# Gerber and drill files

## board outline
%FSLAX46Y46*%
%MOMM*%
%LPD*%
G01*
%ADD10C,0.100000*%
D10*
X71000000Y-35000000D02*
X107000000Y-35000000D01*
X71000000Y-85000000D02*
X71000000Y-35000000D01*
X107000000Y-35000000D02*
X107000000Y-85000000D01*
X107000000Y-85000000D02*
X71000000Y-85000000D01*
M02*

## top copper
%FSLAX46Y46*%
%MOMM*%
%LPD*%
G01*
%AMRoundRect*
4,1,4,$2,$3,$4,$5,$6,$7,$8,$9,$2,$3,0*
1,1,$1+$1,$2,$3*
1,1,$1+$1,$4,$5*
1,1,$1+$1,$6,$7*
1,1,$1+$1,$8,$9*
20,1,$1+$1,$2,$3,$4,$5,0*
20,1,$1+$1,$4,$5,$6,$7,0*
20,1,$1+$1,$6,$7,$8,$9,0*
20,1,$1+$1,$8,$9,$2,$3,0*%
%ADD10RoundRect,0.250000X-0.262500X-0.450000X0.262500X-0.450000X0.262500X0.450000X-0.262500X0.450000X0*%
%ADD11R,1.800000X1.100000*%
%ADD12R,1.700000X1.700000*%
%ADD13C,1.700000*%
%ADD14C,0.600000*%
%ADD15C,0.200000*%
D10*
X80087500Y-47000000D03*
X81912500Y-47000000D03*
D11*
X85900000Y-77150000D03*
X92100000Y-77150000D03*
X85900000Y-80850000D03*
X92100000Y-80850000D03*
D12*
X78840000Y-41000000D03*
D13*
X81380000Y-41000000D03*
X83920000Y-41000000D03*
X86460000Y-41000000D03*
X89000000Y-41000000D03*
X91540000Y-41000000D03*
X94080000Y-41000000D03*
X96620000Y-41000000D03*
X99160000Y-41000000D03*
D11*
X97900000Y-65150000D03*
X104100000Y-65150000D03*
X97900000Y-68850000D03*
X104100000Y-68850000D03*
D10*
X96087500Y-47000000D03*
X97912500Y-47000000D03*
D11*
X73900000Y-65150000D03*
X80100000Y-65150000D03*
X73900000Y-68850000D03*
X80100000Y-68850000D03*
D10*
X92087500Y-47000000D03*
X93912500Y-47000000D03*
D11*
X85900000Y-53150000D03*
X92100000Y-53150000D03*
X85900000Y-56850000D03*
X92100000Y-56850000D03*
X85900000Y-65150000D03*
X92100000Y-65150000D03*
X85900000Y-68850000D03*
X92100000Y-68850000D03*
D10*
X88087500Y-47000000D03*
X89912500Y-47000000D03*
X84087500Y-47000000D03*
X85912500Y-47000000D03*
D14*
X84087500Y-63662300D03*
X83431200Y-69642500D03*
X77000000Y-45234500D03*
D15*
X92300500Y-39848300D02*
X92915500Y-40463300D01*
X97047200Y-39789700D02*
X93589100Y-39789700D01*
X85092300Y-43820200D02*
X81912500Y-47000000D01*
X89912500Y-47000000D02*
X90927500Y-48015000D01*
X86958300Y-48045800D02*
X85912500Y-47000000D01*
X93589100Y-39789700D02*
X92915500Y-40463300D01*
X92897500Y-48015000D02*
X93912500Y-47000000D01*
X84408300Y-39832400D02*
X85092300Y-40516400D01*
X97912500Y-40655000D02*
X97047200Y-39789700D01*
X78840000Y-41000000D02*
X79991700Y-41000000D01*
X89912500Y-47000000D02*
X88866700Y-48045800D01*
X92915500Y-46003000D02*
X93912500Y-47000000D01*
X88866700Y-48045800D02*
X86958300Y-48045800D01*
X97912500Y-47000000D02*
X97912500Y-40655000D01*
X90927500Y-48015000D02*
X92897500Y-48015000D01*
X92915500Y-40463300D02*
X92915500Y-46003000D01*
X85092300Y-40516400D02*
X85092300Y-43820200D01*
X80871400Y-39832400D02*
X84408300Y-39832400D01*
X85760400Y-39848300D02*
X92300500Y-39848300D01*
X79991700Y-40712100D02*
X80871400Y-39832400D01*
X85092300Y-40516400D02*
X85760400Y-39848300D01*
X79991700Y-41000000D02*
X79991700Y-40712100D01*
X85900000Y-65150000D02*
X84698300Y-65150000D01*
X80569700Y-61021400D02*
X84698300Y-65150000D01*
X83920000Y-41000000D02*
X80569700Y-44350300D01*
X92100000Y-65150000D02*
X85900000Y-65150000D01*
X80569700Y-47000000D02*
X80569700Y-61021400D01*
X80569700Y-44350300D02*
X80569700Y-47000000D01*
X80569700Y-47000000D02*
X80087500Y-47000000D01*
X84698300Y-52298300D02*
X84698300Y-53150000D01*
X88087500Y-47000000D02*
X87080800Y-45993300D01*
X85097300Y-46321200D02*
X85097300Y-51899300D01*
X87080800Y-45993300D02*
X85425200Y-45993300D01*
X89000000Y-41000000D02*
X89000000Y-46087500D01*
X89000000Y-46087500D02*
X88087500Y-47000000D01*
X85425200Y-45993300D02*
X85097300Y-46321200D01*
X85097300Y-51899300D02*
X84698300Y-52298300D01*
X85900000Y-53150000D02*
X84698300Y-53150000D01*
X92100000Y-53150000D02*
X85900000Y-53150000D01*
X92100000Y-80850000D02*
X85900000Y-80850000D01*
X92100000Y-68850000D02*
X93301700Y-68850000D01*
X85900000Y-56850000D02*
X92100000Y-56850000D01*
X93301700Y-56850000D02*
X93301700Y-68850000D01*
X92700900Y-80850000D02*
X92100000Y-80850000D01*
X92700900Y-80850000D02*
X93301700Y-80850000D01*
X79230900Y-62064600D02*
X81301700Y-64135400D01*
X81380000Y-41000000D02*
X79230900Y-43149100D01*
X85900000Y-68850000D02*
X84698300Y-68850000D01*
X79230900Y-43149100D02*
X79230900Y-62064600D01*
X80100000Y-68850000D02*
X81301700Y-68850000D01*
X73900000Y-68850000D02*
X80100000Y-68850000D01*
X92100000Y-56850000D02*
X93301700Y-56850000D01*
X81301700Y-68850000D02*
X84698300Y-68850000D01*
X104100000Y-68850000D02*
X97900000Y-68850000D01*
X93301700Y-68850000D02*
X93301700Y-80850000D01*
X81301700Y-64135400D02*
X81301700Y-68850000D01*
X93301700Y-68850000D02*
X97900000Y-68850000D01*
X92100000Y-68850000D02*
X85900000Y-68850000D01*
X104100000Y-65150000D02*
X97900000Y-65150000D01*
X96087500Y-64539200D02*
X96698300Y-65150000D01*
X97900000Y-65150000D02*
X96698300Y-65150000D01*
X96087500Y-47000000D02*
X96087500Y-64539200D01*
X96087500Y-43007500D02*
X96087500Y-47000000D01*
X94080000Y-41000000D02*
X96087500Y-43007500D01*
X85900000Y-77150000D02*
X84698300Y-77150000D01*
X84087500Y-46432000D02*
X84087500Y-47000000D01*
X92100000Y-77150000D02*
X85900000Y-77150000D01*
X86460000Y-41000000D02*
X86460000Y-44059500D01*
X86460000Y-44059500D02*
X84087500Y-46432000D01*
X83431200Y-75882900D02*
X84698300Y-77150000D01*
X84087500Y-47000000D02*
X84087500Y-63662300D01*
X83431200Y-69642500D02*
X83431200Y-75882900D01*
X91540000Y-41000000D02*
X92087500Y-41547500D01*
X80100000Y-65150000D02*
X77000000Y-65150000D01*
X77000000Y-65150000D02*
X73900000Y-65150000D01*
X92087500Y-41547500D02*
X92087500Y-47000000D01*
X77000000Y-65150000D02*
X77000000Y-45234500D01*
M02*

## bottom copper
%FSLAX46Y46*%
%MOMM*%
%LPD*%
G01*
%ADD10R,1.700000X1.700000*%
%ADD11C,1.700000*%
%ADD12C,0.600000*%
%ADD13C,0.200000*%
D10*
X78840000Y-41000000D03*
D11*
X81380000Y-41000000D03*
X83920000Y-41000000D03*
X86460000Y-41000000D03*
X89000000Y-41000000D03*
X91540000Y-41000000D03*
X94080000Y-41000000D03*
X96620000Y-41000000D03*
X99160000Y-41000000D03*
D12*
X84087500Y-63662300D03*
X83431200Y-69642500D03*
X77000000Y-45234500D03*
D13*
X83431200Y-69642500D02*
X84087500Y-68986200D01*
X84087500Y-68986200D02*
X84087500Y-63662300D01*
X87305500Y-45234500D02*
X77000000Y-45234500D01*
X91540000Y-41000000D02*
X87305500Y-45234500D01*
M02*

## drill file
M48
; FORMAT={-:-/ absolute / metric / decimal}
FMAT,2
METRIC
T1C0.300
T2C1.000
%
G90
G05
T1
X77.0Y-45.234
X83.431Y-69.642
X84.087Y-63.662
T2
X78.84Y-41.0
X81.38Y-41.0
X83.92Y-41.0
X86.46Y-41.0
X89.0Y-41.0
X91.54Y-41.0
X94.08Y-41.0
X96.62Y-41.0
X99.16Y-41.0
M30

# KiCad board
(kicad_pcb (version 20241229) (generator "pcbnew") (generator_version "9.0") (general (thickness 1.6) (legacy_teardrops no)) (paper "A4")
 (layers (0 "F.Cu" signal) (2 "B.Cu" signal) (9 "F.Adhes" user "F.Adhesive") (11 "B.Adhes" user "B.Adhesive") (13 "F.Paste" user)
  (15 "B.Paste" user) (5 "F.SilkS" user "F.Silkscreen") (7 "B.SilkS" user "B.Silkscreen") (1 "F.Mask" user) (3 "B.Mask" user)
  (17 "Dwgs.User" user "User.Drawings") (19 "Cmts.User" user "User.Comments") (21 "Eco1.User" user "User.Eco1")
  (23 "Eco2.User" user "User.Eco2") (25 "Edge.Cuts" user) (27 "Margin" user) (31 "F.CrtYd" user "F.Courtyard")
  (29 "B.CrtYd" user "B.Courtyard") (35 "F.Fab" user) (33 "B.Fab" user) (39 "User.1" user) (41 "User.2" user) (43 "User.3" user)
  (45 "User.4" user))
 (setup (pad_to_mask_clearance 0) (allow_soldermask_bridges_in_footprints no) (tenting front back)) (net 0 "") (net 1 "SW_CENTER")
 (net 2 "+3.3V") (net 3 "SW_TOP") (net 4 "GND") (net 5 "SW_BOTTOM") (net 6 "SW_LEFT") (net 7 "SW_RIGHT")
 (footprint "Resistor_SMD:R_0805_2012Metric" (layer "F.Cu") (at 81 47)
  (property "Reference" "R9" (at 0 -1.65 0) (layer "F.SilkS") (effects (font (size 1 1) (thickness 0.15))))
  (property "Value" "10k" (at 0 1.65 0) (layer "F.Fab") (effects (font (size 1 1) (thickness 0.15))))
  (pad "1" smd roundrect (at -0.9125 0) (size 1.025 1.4) (layers "F.Cu" "F.Mask" "F.Paste") (roundrect_rratio 0.243902) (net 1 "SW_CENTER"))
  (pad "2" smd roundrect (at 0.9125 0) (size 1.025 1.4) (layers "F.Cu" "F.Mask" "F.Paste") (roundrect_rratio 0.243902) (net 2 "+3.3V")))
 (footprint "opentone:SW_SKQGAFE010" (layer "F.Cu") (at 89 79)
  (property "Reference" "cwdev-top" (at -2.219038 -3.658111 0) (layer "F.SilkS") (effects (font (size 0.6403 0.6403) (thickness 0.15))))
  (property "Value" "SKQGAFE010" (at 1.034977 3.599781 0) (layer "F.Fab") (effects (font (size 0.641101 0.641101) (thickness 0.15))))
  (pad "1" smd rect (at -3.1 -1.85) (size 1.8 1.1) (layers "F.Cu" "F.Mask" "F.Paste") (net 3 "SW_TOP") (solder_mask_margin 0.102))
  (pad "2" smd rect (at 3.1 -1.85) (size 1.8 1.1) (layers "F.Cu" "F.Mask" "F.Paste") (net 3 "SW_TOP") (solder_mask_margin 0.102))
  (pad "3" smd rect (at -3.1 1.85) (size 1.8 1.1) (layers "F.Cu" "F.Mask" "F.Paste") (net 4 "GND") (solder_mask_margin 0.102))
  (pad "4" smd rect (at 3.1 1.85) (size 1.8 1.1) (layers "F.Cu" "F.Mask" "F.Paste") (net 4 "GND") (solder_mask_margin 0.102))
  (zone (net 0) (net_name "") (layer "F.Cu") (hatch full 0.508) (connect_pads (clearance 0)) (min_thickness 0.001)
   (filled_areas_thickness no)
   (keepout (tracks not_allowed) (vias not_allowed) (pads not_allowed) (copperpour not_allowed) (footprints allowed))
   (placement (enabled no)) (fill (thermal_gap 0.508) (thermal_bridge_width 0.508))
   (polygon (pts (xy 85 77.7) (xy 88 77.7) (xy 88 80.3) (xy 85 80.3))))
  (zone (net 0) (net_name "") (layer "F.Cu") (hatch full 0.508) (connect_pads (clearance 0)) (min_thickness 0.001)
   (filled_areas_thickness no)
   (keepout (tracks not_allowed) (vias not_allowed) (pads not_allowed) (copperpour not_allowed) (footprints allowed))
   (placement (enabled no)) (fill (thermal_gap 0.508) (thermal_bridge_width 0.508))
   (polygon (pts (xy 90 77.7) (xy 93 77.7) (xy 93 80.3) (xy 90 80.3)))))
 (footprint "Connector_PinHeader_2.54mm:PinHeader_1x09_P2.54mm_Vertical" (layer "F.Cu") (at 78.84 41 90)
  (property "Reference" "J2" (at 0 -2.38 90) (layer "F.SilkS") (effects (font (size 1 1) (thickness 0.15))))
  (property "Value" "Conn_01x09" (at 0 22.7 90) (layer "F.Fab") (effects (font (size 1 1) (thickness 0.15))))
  (pad "1" thru_hole rect (at 0 0 90) (size 1.7 1.7) (drill 1) (layers "*.Cu" "*.Mask") (remove_unused_layers no) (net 2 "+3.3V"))
  (pad "2" thru_hole circle (at 0 2.54 90) (size 1.7 1.7) (drill 1) (layers "*.Cu" "*.Mask") (remove_unused_layers no) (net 4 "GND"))
  (pad "3" thru_hole circle (at 0 5.08 90) (size 1.7 1.7) (drill 1) (layers "*.Cu" "*.Mask") (remove_unused_layers no) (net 1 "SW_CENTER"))
  (pad "4" thru_hole circle (at 0 7.62 90) (size 1.7 1.7) (drill 1) (layers "*.Cu" "*.Mask") (remove_unused_layers no) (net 3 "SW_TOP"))
  (pad "5" thru_hole circle (at 0 10.16 90) (size 1.7 1.7) (drill 1) (layers "*.Cu" "*.Mask") (remove_unused_layers no) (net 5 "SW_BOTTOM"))
  (pad "6" thru_hole circle (at 0 12.7 90) (size 1.7 1.7) (drill 1) (layers "*.Cu" "*.Mask") (remove_unused_layers no) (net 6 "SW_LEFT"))
  (pad "7" thru_hole circle (at 0 15.24 90) (size 1.7 1.7) (drill 1) (layers "*.Cu" "*.Mask") (remove_unused_layers no) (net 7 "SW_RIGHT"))
  (pad "8" thru_hole circle (at 0 17.78 90) (size 1.7 1.7) (drill 1) (layers "*.Cu" "*.Mask") (remove_unused_layers no))
  (pad "9" thru_hole circle (at 0 20.32 90) (size 1.7 1.7) (drill 1) (layers "*.Cu" "*.Mask") (remove_unused_layers no)))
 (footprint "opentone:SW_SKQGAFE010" (layer "F.Cu") (at 101 67)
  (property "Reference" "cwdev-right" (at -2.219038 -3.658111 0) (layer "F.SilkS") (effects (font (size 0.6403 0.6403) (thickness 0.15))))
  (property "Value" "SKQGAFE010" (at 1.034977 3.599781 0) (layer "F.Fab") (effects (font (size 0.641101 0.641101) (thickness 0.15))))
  (pad "1" smd rect (at -3.1 -1.85) (size 1.8 1.1) (layers "F.Cu" "F.Mask" "F.Paste") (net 7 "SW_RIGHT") (solder_mask_margin 0.102))
  (pad "2" smd rect (at 3.1 -1.85) (size 1.8 1.1) (layers "F.Cu" "F.Mask" "F.Paste") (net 7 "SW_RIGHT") (solder_mask_margin 0.102))
  (pad "3" smd rect (at -3.1 1.85) (size 1.8 1.1) (layers "F.Cu" "F.Mask" "F.Paste") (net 4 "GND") (solder_mask_margin 0.102))
  (pad "4" smd rect (at 3.1 1.85) (size 1.8 1.1) (layers "F.Cu" "F.Mask" "F.Paste") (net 4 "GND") (solder_mask_margin 0.102))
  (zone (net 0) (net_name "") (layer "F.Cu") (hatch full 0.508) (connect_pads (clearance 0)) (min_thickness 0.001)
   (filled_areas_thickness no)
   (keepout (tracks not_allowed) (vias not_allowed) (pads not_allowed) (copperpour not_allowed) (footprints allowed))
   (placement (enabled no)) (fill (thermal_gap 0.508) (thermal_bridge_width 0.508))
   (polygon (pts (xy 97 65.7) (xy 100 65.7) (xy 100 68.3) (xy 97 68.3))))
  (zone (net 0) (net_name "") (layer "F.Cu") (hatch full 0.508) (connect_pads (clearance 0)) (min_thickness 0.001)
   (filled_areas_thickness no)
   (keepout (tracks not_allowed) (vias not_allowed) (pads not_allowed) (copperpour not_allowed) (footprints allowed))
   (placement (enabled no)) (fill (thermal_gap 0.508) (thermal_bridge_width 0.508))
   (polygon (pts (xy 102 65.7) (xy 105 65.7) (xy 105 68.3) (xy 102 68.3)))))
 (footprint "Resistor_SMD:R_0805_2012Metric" (layer "F.Cu") (at 97 47)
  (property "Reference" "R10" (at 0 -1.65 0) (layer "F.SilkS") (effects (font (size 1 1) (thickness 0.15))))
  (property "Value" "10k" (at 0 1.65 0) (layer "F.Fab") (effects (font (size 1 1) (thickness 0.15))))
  (pad "1" smd roundrect (at -0.9125 0) (size 1.025 1.4) (layers "F.Cu" "F.Mask" "F.Paste") (roundrect_rratio 0.243902) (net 7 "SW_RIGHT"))
  (pad "2" smd roundrect (at 0.9125 0) (size 1.025 1.4) (layers "F.Cu" "F.Mask" "F.Paste") (roundrect_rratio 0.243902) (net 2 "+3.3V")))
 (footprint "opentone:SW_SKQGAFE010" (layer "F.Cu") (at 77 67)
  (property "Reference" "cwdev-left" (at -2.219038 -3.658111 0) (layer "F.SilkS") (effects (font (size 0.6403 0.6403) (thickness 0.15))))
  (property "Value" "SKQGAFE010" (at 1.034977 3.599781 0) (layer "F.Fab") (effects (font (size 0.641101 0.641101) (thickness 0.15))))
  (pad "1" smd rect (at -3.1 -1.85) (size 1.8 1.1) (layers "F.Cu" "F.Mask" "F.Paste") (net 6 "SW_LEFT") (solder_mask_margin 0.102))
  (pad "2" smd rect (at 3.1 -1.85) (size 1.8 1.1) (layers "F.Cu" "F.Mask" "F.Paste") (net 6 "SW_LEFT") (solder_mask_margin 0.102))
  (pad "3" smd rect (at -3.1 1.85) (size 1.8 1.1) (layers "F.Cu" "F.Mask" "F.Paste") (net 4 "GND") (solder_mask_margin 0.102))
  (pad "4" smd rect (at 3.1 1.85) (size 1.8 1.1) (layers "F.Cu" "F.Mask" "F.Paste") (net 4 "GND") (solder_mask_margin 0.102))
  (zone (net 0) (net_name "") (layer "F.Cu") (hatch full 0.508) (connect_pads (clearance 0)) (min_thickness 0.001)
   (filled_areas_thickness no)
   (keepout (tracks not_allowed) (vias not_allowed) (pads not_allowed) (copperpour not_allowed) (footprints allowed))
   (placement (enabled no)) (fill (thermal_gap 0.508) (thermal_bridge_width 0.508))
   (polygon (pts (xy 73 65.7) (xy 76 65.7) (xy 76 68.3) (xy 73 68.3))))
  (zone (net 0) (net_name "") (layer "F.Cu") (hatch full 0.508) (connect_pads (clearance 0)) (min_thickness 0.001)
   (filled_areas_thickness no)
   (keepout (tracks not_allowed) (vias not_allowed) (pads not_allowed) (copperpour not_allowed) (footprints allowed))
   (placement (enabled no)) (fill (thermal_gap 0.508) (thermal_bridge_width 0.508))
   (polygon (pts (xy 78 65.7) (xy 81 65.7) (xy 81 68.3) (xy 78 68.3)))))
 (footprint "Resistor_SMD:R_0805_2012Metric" (layer "F.Cu") (at 93 47)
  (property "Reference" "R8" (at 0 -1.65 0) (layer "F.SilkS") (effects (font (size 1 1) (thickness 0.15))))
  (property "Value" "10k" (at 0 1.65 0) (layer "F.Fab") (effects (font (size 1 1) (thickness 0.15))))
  (pad "1" smd roundrect (at -0.9125 0) (size 1.025 1.4) (layers "F.Cu" "F.Mask" "F.Paste") (roundrect_rratio 0.243902) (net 6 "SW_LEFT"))
  (pad "2" smd roundrect (at 0.9125 0) (size 1.025 1.4) (layers "F.Cu" "F.Mask" "F.Paste") (roundrect_rratio 0.243902) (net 2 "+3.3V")))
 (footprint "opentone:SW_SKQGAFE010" (layer "F.Cu") (at 89 55)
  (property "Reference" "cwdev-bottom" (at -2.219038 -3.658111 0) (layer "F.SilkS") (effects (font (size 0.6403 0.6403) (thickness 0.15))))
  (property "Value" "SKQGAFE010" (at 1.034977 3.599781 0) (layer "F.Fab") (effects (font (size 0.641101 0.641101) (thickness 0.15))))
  (pad "1" smd rect (at -3.1 -1.85) (size 1.8 1.1) (layers "F.Cu" "F.Mask" "F.Paste") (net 5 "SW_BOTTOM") (solder_mask_margin 0.102))
  (pad "2" smd rect (at 3.1 -1.85) (size 1.8 1.1) (layers "F.Cu" "F.Mask" "F.Paste") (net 5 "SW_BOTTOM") (solder_mask_margin 0.102))
  (pad "3" smd rect (at -3.1 1.85) (size 1.8 1.1) (layers "F.Cu" "F.Mask" "F.Paste") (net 4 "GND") (solder_mask_margin 0.102))
  (pad "4" smd rect (at 3.1 1.85) (size 1.8 1.1) (layers "F.Cu" "F.Mask" "F.Paste") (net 4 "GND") (solder_mask_margin 0.102))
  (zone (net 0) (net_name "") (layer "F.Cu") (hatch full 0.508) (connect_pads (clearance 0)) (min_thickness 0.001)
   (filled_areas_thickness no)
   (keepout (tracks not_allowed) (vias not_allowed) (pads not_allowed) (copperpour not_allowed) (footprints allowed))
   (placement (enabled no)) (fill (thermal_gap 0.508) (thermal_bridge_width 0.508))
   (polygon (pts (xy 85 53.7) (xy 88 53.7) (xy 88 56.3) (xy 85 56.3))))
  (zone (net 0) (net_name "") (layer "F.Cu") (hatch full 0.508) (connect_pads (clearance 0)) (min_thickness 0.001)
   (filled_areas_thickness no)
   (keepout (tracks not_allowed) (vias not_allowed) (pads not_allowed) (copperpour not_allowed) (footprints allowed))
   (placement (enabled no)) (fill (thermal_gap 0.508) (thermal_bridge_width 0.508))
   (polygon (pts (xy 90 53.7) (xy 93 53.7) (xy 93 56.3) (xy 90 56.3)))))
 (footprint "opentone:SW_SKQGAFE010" (layer "F.Cu") (at 89 67)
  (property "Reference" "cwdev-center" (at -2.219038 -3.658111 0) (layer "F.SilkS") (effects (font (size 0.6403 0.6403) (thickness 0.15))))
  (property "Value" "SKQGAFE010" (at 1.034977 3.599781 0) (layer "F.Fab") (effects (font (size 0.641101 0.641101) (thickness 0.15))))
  (pad "1" smd rect (at -3.1 -1.85) (size 1.8 1.1) (layers "F.Cu" "F.Mask" "F.Paste") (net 1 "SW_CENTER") (solder_mask_margin 0.102))
  (pad "2" smd rect (at 3.1 -1.85) (size 1.8 1.1) (layers "F.Cu" "F.Mask" "F.Paste") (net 1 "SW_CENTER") (solder_mask_margin 0.102))
  (pad "3" smd rect (at -3.1 1.85) (size 1.8 1.1) (layers "F.Cu" "F.Mask" "F.Paste") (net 4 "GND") (solder_mask_margin 0.102))
  (pad "4" smd rect (at 3.1 1.85) (size 1.8 1.1) (layers "F.Cu" "F.Mask" "F.Paste") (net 4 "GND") (solder_mask_margin 0.102))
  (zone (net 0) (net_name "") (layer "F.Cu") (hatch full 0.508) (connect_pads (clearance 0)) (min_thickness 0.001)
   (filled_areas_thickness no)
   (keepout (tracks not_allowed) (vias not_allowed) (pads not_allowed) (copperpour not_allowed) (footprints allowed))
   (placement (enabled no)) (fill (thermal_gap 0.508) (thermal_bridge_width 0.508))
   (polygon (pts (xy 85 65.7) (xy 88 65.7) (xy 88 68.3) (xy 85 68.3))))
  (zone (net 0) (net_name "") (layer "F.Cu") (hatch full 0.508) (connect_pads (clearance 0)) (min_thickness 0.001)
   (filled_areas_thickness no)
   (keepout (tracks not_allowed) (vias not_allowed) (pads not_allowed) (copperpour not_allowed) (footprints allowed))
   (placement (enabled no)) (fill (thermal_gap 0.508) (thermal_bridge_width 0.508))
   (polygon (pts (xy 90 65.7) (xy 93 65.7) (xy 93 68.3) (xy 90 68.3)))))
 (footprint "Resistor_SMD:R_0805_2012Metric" (layer "F.Cu") (at 89 47)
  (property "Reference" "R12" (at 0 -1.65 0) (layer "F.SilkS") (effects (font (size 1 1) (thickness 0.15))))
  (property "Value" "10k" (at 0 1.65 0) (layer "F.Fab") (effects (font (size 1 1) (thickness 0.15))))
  (pad "1" smd roundrect (at -0.9125 0) (size 1.025 1.4) (layers "F.Cu" "F.Mask" "F.Paste") (roundrect_rratio 0.243902) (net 5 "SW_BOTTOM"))
  (pad "2" smd roundrect (at 0.9125 0) (size 1.025 1.4) (layers "F.Cu" "F.Mask" "F.Paste") (roundrect_rratio 0.243902) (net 2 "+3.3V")))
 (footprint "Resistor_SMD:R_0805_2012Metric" (layer "F.Cu") (at 85 47)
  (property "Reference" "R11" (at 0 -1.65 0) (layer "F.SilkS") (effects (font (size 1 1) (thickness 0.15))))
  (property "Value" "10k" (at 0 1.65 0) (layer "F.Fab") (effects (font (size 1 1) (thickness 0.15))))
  (pad "1" smd roundrect (at -0.9125 0) (size 1.025 1.4) (layers "F.Cu" "F.Mask" "F.Paste") (roundrect_rratio 0.243902) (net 3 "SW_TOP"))
  (pad "2" smd roundrect (at 0.9125 0) (size 1.025 1.4) (layers "F.Cu" "F.Mask" "F.Paste") (roundrect_rratio 0.243902) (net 2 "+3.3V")))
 (gr_line (start 71 35) (end 107 35) (stroke (width 0.1) (type default)) (layer "Edge.Cuts"))
 (gr_line (start 71 85) (end 71 35) (stroke (width 0.1) (type default)) (layer "Edge.Cuts"))
 (gr_line (start 107 35) (end 107 85) (stroke (width 0.1) (type default)) (layer "Edge.Cuts"))
 (gr_line (start 107 85) (end 71 85) (stroke (width 0.1) (type default)) (layer "Edge.Cuts"))
 (segment (start 92.3005 39.8483) (end 92.9155 40.4633) (width 0.2) (layer "F.Cu") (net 2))
 (segment (start 97.0472 39.7897) (end 93.5891 39.7897) (width 0.2) (layer "F.Cu") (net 2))
 (segment (start 85.0923 43.8202) (end 81.9125 47) (width 0.2) (layer "F.Cu") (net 2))
 (segment (start 89.9125 47) (end 90.9275 48.015) (width 0.2) (layer "F.Cu") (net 2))
 (segment (start 86.9583 48.0458) (end 85.9125 47) (width 0.2) (layer "F.Cu") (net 2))
 (segment (start 93.5891 39.7897) (end 92.9155 40.4633) (width 0.2) (layer "F.Cu") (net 2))
 (segment (start 92.8975 48.015) (end 93.9125 47) (width 0.2) (layer "F.Cu") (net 2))
 (segment (start 84.4083 39.8324) (end 85.0923 40.5164) (width 0.2) (layer "F.Cu") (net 2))
 (segment (start 97.9125 40.655) (end 97.0472 39.7897) (width 0.2) (layer "F.Cu") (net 2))
 (segment (start 78.84 41) (end 79.9917 41) (width 0.2) (layer "F.Cu") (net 2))
 (segment (start 89.9125 47) (end 88.8667 48.0458) (width 0.2) (layer "F.Cu") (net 2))
 (segment (start 92.9155 46.003) (end 93.9125 47) (width 0.2) (layer "F.Cu") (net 2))
 (segment (start 88.8667 48.0458) (end 86.9583 48.0458) (width 0.2) (layer "F.Cu") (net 2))
 (segment (start 97.9125 47) (end 97.9125 40.655) (width 0.2) (layer "F.Cu") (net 2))
 (segment (start 90.9275 48.015) (end 92.8975 48.015) (width 0.2) (layer "F.Cu") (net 2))
 (segment (start 92.9155 40.4633) (end 92.9155 46.003) (width 0.2) (layer "F.Cu") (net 2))
 (segment (start 85.0923 40.5164) (end 85.0923 43.8202) (width 0.2) (layer "F.Cu") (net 2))
 (segment (start 80.8714 39.8324) (end 84.4083 39.8324) (width 0.2) (layer "F.Cu") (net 2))
 (segment (start 85.7604 39.8483) (end 92.3005 39.8483) (width 0.2) (layer "F.Cu") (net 2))
 (segment (start 79.9917 40.7121) (end 80.8714 39.8324) (width 0.2) (layer "F.Cu") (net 2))
 (segment (start 85.0923 40.5164) (end 85.7604 39.8483) (width 0.2) (layer "F.Cu") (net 2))
 (segment (start 79.9917 41) (end 79.9917 40.7121) (width 0.2) (layer "F.Cu") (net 2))
 (segment (start 85.9 65.15) (end 84.6983 65.15) (width 0.2) (layer "F.Cu") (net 1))
 (segment (start 80.5697 61.0214) (end 84.6983 65.15) (width 0.2) (layer "F.Cu") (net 1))
 (segment (start 83.92 41) (end 80.5697 44.3503) (width 0.2) (layer "F.Cu") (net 1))
 (segment (start 92.1 65.15) (end 85.9 65.15) (width 0.2) (layer "F.Cu") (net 1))
 (segment (start 80.5697 47) (end 80.5697 61.0214) (width 0.2) (layer "F.Cu") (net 1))
 (segment (start 80.5697 44.3503) (end 80.5697 47) (width 0.2) (layer "F.Cu") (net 1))
 (segment (start 80.5697 47) (end 80.0875 47) (width 0.2) (layer "F.Cu") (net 1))
 (segment (start 84.6983 52.2983) (end 84.6983 53.15) (width 0.2) (layer "F.Cu") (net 5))
 (segment (start 88.0875 47) (end 87.0808 45.9933) (width 0.2) (layer "F.Cu") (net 5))
 (segment (start 85.0973 46.3212) (end 85.0973 51.8993) (width 0.2) (layer "F.Cu") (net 5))
 (segment (start 87.0808 45.9933) (end 85.4252 45.9933) (width 0.2) (layer "F.Cu") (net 5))
 (segment (start 89 41) (end 89 46.0875) (width 0.2) (layer "F.Cu") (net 5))
 (segment (start 89 46.0875) (end 88.0875 47) (width 0.2) (layer "F.Cu") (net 5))
 (segment (start 85.4252 45.9933) (end 85.0973 46.3212) (width 0.2) (layer "F.Cu") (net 5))
 (segment (start 85.0973 51.8993) (end 84.6983 52.2983) (width 0.2) (layer "F.Cu") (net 5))
 (segment (start 85.9 53.15) (end 84.6983 53.15) (width 0.2) (layer "F.Cu") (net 5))
 (segment (start 92.1 53.15) (end 85.9 53.15) (width 0.2) (layer "F.Cu") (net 5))
 (segment (start 92.1 80.85) (end 85.9 80.85) (width 0.2) (layer "F.Cu") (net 4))
 (segment (start 92.1 68.85) (end 93.3017 68.85) (width 0.2) (layer "F.Cu") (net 4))
 (segment (start 85.9 56.85) (end 92.1 56.85) (width 0.2) (layer "F.Cu") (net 4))
 (segment (start 93.3017 56.85) (end 93.3017 68.85) (width 0.2) (layer "F.Cu") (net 4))
 (segment (start 92.7009 80.85) (end 92.1 80.85) (width 0.2) (layer "F.Cu") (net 4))
 (segment (start 92.7009 80.85) (end 93.3017 80.85) (width 0.2) (layer "F.Cu") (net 4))
 (segment (start 79.2309 62.0646) (end 81.3017 64.1354) (width 0.2) (layer "F.Cu") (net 4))
 (segment (start 81.38 41) (end 79.2309 43.1491) (width 0.2) (layer "F.Cu") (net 4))
 (segment (start 85.9 68.85) (end 84.6983 68.85) (width 0.2) (layer "F.Cu") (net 4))
 (segment (start 79.2309 43.1491) (end 79.2309 62.0646) (width 0.2) (layer "F.Cu") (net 4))
 (segment (start 80.1 68.85) (end 81.3017 68.85) (width 0.2) (layer "F.Cu") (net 4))
 (segment (start 73.9 68.85) (end 80.1 68.85) (width 0.2) (layer "F.Cu") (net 4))
 (segment (start 92.1 56.85) (end 93.3017 56.85) (width 0.2) (layer "F.Cu") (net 4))
 (segment (start 81.3017 68.85) (end 84.6983 68.85) (width 0.2) (layer "F.Cu") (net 4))
 (segment (start 104.1 68.85) (end 97.9 68.85) (width 0.2) (layer "F.Cu") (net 4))
 (segment (start 93.3017 68.85) (end 93.3017 80.85) (width 0.2) (layer "F.Cu") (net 4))
 (segment (start 81.3017 64.1354) (end 81.3017 68.85) (width 0.2) (layer "F.Cu") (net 4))
 (segment (start 93.3017 68.85) (end 97.9 68.85) (width 0.2) (layer "F.Cu") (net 4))
 (segment (start 92.1 68.85) (end 85.9 68.85) (width 0.2) (layer "F.Cu") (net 4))
 (segment (start 104.1 65.15) (end 97.9 65.15) (width 0.2) (layer "F.Cu") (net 7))
 (segment (start 96.0875 64.5392) (end 96.6983 65.15) (width 0.2) (layer "F.Cu") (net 7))
 (segment (start 97.9 65.15) (end 96.6983 65.15) (width 0.2) (layer "F.Cu") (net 7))
 (segment (start 96.0875 47) (end 96.0875 64.5392) (width 0.2) (layer "F.Cu") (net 7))
 (segment (start 96.0875 43.0075) (end 96.0875 47) (width 0.2) (layer "F.Cu") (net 7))
 (segment (start 94.08 41) (end 96.0875 43.0075) (width 0.2) (layer "F.Cu") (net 7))
 (segment (start 85.9 77.15) (end 84.6983 77.15) (width 0.2) (layer "F.Cu") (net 3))
 (segment (start 84.0875 46.432) (end 84.0875 47) (width 0.2) (layer "F.Cu") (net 3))
 (segment (start 92.1 77.15) (end 85.9 77.15) (width 0.2) (layer "F.Cu") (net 3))
 (segment (start 86.46 41) (end 86.46 44.0595) (width 0.2) (layer "F.Cu") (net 3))
 (segment (start 86.46 44.0595) (end 84.0875 46.432) (width 0.2) (layer "F.Cu") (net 3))
 (segment (start 83.4312 75.8829) (end 84.6983 77.15) (width 0.2) (layer "F.Cu") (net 3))
 (segment (start 84.0875 47) (end 84.0875 63.6623) (width 0.2) (layer "F.Cu") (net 3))
 (segment (start 83.4312 69.6425) (end 83.4312 75.8829) (width 0.2) (layer "F.Cu") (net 3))
 (via (at 84.0875 63.6623) (size 0.6) (drill 0.3) (layers "F.Cu" "B.Cu") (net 3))
 (via (at 83.4312 69.6425) (size 0.6) (drill 0.3) (layers "F.Cu" "B.Cu") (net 3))
 (segment (start 83.4312 69.6425) (end 84.0875 68.9862) (width 0.2) (layer "B.Cu") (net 3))
 (segment (start 84.0875 68.9862) (end 84.0875 63.6623) (width 0.2) (layer "B.Cu") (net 3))
 (segment (start 91.54 41) (end 92.0875 41.5475) (width 0.2) (layer "F.Cu") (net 6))
 (segment (start 80.1 65.15) (end 77 65.15) (width 0.2) (layer "F.Cu") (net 6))
 (segment (start 77 65.15) (end 73.9 65.15) (width 0.2) (layer "F.Cu") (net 6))
 (segment (start 92.0875 41.5475) (end 92.0875 47) (width 0.2) (layer "F.Cu") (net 6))
 (segment (start 77 65.15) (end 77 45.2345) (width 0.2) (layer "F.Cu") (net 6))
 (via (at 77 45.2345) (size 0.6) (drill 0.3) (layers "F.Cu" "B.Cu") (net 6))
 (segment (start 87.3055 45.2345) (end 77 45.2345) (width 0.2) (layer "B.Cu") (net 6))
 (segment (start 91.54 41) (end 87.3055 45.2345) (width 0.2) (layer "B.Cu") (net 6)))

